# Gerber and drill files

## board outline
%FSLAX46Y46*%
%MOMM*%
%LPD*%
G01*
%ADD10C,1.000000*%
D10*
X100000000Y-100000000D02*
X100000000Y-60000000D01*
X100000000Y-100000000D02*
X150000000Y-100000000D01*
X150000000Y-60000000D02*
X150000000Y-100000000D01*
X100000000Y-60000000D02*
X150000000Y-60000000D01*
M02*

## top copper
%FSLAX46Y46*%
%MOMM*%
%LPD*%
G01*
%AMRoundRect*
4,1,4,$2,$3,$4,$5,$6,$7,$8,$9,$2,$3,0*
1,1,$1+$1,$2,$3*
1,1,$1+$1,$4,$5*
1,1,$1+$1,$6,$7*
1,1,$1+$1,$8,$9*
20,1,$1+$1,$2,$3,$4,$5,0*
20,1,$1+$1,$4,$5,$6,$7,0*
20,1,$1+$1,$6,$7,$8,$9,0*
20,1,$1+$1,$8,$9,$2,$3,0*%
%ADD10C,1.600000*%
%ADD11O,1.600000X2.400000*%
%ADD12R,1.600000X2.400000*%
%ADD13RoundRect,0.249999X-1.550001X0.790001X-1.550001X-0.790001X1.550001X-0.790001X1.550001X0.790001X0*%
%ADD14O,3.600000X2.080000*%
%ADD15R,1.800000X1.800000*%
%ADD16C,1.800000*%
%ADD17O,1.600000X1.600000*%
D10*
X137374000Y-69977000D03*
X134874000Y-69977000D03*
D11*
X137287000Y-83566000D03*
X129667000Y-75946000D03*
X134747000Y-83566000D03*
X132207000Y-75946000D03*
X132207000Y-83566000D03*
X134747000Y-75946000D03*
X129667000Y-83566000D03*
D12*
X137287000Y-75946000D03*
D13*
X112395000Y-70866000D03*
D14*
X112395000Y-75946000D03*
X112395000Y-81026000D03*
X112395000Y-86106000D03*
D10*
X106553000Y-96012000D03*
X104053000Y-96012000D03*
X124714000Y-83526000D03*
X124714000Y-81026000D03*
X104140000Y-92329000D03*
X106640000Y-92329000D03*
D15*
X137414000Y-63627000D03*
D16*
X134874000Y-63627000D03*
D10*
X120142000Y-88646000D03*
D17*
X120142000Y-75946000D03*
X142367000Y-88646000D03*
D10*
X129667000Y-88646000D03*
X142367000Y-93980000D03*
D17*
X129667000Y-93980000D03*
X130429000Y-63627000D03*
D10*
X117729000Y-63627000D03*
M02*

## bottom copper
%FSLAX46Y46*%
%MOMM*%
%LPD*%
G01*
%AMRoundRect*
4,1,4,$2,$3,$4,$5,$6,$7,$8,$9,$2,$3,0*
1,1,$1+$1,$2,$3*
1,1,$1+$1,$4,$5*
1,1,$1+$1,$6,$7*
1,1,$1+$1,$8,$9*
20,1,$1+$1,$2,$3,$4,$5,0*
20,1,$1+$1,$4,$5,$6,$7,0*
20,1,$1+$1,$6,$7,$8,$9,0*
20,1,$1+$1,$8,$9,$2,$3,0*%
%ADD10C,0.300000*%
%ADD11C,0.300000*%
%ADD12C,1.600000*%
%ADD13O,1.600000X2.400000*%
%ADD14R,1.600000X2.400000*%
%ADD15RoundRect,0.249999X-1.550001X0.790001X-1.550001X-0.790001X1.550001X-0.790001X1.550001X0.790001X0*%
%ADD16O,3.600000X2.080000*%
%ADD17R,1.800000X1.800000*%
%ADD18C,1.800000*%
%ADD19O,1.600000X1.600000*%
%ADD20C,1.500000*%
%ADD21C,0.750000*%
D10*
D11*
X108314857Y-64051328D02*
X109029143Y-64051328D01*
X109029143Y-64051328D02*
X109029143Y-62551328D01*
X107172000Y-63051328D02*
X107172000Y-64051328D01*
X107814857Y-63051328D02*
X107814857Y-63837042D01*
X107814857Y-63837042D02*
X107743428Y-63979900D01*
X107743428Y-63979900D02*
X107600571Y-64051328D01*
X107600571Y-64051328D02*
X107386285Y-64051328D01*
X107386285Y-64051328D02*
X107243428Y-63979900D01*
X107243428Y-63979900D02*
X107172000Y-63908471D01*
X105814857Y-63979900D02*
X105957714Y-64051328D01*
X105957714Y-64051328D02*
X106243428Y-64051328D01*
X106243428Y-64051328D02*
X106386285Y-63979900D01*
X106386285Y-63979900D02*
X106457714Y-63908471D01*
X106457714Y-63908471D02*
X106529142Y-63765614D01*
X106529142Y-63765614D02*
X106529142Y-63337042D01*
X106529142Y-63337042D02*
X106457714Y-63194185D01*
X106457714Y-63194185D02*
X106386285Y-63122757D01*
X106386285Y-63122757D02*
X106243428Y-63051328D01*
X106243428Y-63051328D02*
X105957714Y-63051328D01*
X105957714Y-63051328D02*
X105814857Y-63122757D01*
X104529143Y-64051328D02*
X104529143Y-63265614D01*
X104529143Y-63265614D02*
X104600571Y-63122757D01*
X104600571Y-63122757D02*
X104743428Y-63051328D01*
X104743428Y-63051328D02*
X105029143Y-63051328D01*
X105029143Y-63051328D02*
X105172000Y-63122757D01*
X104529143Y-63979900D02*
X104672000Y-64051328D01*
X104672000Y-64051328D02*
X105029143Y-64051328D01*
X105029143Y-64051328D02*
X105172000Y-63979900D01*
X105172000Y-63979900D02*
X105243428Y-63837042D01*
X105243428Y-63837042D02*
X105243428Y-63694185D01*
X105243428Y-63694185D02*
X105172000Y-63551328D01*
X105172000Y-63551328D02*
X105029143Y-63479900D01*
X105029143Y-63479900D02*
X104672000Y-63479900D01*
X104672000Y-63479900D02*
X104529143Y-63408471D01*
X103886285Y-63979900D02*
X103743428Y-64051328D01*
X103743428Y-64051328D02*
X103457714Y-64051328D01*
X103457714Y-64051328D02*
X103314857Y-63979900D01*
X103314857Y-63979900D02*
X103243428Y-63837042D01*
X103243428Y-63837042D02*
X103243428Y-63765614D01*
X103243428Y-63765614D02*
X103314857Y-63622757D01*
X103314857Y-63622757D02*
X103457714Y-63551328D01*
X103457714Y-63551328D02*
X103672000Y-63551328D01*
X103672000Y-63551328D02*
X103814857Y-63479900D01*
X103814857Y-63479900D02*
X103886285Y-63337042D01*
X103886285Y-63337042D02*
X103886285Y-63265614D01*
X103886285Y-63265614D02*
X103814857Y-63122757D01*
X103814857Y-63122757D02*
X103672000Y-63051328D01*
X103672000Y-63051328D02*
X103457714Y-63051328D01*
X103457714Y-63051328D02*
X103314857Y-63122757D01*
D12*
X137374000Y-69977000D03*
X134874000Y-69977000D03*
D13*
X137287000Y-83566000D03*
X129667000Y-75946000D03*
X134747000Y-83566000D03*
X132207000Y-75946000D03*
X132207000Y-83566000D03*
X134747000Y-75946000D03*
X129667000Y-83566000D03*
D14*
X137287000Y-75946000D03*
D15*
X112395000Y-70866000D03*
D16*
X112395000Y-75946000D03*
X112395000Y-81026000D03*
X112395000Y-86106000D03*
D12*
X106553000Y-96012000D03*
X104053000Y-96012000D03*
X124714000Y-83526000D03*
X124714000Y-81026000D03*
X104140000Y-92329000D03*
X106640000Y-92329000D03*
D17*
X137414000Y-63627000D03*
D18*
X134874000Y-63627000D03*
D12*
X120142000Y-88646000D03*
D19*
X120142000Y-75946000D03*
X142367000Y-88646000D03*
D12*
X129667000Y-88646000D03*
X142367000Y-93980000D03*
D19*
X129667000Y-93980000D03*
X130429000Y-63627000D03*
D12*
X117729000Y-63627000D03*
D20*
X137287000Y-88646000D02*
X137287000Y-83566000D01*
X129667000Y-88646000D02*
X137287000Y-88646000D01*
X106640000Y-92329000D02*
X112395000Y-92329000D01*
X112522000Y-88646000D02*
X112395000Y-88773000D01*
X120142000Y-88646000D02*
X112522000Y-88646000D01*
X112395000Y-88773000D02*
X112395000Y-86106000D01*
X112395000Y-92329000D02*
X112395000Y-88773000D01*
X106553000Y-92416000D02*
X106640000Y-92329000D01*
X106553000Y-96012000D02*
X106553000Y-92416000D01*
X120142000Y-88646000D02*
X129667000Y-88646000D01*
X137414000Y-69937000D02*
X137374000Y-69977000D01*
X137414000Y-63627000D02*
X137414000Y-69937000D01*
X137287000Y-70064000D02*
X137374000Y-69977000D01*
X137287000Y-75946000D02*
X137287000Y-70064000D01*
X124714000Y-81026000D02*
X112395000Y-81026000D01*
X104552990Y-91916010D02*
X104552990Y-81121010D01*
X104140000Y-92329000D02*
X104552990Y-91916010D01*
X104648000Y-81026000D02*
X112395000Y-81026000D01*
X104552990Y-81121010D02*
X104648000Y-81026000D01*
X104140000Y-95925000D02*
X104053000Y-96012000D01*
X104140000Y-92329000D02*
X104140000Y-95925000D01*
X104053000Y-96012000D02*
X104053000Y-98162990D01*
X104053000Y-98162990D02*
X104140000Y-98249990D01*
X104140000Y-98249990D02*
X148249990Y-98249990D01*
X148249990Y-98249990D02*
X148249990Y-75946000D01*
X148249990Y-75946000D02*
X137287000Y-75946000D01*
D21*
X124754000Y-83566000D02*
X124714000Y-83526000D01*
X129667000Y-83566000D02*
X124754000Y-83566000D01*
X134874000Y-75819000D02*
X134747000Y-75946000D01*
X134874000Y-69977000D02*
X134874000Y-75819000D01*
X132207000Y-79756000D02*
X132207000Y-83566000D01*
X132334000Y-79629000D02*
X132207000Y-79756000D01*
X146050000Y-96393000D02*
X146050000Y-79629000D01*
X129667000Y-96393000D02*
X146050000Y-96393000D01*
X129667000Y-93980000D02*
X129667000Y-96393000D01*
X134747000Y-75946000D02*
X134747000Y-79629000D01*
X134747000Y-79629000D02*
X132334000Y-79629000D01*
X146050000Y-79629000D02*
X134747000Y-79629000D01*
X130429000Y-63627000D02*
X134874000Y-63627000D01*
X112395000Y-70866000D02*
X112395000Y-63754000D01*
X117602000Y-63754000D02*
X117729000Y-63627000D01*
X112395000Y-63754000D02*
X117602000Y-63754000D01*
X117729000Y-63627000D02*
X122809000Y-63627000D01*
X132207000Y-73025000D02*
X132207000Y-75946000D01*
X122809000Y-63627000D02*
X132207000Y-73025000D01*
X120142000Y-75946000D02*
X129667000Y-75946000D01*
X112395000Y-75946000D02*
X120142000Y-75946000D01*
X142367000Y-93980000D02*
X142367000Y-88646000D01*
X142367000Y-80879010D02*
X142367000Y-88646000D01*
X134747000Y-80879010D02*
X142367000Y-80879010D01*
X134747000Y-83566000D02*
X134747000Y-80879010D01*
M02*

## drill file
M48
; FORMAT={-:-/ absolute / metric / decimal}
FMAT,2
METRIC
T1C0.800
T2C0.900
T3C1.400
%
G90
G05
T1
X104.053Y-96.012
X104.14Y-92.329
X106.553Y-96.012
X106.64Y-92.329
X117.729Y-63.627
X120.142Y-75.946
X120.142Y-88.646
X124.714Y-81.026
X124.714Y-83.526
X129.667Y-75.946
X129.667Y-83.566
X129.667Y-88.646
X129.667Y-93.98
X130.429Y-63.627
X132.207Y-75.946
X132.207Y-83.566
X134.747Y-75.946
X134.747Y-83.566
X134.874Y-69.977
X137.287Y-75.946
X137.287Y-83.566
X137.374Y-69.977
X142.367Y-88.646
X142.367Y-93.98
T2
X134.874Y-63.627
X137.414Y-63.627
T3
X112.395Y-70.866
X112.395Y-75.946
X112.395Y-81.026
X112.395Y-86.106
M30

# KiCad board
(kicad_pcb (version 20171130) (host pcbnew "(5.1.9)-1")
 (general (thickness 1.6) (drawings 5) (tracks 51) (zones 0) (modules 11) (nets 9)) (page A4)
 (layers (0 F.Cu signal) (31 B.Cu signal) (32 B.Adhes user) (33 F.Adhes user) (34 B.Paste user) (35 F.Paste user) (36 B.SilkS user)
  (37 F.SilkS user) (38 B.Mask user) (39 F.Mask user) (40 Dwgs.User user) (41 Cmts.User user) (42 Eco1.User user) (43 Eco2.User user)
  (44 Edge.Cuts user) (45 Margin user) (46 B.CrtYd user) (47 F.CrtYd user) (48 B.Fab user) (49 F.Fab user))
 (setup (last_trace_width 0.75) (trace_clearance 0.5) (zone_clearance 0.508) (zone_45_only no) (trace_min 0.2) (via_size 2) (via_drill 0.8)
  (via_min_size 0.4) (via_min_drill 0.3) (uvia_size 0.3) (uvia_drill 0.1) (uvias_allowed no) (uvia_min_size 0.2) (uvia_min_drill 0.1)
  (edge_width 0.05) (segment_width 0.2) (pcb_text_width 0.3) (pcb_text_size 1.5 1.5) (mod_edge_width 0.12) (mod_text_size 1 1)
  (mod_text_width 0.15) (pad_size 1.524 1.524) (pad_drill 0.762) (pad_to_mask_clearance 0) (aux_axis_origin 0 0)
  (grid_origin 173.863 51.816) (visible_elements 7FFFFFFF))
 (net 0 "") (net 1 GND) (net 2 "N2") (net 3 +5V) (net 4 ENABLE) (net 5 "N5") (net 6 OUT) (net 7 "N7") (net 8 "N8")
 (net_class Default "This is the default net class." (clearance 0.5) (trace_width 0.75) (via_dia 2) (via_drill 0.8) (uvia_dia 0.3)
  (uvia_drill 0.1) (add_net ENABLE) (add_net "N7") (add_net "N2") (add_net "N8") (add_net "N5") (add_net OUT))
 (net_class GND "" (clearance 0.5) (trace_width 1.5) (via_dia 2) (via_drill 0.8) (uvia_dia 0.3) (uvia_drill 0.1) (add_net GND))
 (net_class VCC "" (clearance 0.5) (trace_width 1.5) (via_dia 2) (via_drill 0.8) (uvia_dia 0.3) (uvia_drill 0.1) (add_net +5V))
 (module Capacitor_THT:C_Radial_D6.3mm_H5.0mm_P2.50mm (layer F.Cu) (at 134.874 69.977)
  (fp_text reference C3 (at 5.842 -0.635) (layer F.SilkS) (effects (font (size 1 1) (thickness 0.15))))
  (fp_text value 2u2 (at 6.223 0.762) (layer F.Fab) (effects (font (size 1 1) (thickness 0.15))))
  (pad 2 thru_hole circle (at 2.5 0) (size 1.6 1.6) (drill 0.8) (layers *.Cu *.Mask) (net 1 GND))
  (pad 1 thru_hole circle (at 0 0) (size 1.6 1.6) (drill 0.8) (layers *.Cu *.Mask) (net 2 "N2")))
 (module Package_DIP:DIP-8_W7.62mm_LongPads (layer F.Cu) (at 137.287 75.946 270)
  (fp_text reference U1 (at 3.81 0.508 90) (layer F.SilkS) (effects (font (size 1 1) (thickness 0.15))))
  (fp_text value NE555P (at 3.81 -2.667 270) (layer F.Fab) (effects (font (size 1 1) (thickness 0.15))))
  (pad 8 thru_hole oval (at 7.62 0 270) (size 2.4 1.6) (drill 0.8) (layers *.Cu *.Mask) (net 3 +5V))
  (pad 4 thru_hole oval (at 0 7.62 270) (size 2.4 1.6) (drill 0.8) (layers *.Cu *.Mask) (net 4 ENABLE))
  (pad 7 thru_hole oval (at 7.62 2.54 270) (size 2.4 1.6) (drill 0.8) (layers *.Cu *.Mask) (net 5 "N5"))
  (pad 3 thru_hole oval (at 0 5.08 270) (size 2.4 1.6) (drill 0.8) (layers *.Cu *.Mask) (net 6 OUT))
  (pad 6 thru_hole oval (at 7.62 5.08 270) (size 2.4 1.6) (drill 0.8) (layers *.Cu *.Mask) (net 2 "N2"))
  (pad 2 thru_hole oval (at 0 2.54 270) (size 2.4 1.6) (drill 0.8) (layers *.Cu *.Mask) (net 2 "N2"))
  (pad 5 thru_hole oval (at 7.62 7.62 270) (size 2.4 1.6) (drill 0.8) (layers *.Cu *.Mask) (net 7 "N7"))
  (pad 1 thru_hole rect (at 0 0 270) (size 2.4 1.6) (drill 0.8) (layers *.Cu *.Mask) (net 1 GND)))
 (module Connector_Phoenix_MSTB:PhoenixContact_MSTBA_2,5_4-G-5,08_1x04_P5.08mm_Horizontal (layer F.Cu) (at 112.395 70.866 270)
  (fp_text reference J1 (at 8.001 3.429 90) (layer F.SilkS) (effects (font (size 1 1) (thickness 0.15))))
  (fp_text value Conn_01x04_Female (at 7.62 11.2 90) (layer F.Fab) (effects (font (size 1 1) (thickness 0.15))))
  (pad 1 thru_hole roundrect (at 0 0 270) (size 2.08 3.6) (drill 1.4) (layers *.Cu *.Mask) (roundrect_rratio 0.120192) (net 6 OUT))
  (pad 2 thru_hole oval (at 5.08 0 270) (size 2.08 3.6) (drill 1.4) (layers *.Cu *.Mask) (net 4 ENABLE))
  (pad 3 thru_hole oval (at 10.16 0 270) (size 2.08 3.6) (drill 1.4) (layers *.Cu *.Mask) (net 1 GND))
  (pad 4 thru_hole oval (at 15.24 0 270) (size 2.08 3.6) (drill 1.4) (layers *.Cu *.Mask) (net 3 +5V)))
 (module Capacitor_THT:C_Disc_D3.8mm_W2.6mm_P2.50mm (layer F.Cu) (at 106.553 96.012 180)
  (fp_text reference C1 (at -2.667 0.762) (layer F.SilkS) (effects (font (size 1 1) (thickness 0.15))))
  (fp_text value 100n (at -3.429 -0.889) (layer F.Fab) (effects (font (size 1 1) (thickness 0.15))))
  (pad 1 thru_hole circle (at 0 0 180) (size 1.6 1.6) (drill 0.8) (layers *.Cu *.Mask) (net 3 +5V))
  (pad 2 thru_hole circle (at 2.5 0 180) (size 1.6 1.6) (drill 0.8) (layers *.Cu *.Mask) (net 1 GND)))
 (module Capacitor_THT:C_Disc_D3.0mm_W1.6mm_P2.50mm (layer F.Cu) (at 124.714 83.526 90)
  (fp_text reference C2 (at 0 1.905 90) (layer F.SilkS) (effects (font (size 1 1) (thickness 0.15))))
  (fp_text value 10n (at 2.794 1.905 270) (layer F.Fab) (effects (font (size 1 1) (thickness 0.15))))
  (pad 1 thru_hole circle (at 0 0 90) (size 1.6 1.6) (drill 0.8) (layers *.Cu *.Mask) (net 7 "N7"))
  (pad 2 thru_hole circle (at 2.5 0 90) (size 1.6 1.6) (drill 0.8) (layers *.Cu *.Mask) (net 1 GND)))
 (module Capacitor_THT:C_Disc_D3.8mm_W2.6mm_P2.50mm (layer F.Cu) (at 106.64 92.329 180)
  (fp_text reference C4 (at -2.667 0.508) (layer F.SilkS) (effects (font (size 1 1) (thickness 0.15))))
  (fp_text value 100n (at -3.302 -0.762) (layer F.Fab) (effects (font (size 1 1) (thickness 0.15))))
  (pad 2 thru_hole circle (at 2.5 0 180) (size 1.6 1.6) (drill 0.8) (layers *.Cu *.Mask) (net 1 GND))
  (pad 1 thru_hole circle (at 0 0 180) (size 1.6 1.6) (drill 0.8) (layers *.Cu *.Mask) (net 3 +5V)))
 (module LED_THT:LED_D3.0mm (layer F.Cu) (at 137.414 63.627 180)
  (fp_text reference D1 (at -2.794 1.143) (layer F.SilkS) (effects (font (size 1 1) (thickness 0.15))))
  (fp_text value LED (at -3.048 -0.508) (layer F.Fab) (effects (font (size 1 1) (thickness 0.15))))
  (pad 1 thru_hole rect (at 0 0 180) (size 1.8 1.8) (drill 0.9) (layers *.Cu *.Mask) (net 1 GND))
  (pad 2 thru_hole circle (at 2.54 0 180) (size 1.8 1.8) (drill 0.9) (layers *.Cu *.Mask) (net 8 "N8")))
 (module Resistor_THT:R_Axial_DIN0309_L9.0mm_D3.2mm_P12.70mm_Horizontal (layer F.Cu) (at 120.142 88.646 90)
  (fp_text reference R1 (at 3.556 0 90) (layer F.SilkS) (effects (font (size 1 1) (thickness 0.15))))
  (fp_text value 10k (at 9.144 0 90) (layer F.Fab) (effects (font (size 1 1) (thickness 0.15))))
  (pad 1 thru_hole circle (at 0 0 90) (size 1.6 1.6) (drill 0.8) (layers *.Cu *.Mask) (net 3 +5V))
  (pad 2 thru_hole oval (at 12.7 0 90) (size 1.6 1.6) (drill 0.8) (layers *.Cu *.Mask) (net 4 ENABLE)))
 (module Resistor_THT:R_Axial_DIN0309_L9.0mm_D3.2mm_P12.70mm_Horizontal (layer F.Cu) (at 129.667 88.646)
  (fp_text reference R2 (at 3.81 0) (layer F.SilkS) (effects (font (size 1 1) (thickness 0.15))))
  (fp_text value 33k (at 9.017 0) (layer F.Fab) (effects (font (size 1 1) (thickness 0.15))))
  (pad 2 thru_hole oval (at 12.7 0) (size 1.6 1.6) (drill 0.8) (layers *.Cu *.Mask) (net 5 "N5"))
  (pad 1 thru_hole circle (at 0 0) (size 1.6 1.6) (drill 0.8) (layers *.Cu *.Mask) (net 3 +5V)))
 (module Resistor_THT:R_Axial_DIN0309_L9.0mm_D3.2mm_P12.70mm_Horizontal (layer F.Cu) (at 142.367 93.98 180)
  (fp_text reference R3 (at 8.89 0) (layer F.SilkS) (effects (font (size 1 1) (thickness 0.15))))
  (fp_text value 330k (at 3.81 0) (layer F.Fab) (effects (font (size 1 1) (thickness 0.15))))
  (pad 1 thru_hole circle (at 0 0 180) (size 1.6 1.6) (drill 0.8) (layers *.Cu *.Mask) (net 5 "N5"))
  (pad 2 thru_hole oval (at 12.7 0 180) (size 1.6 1.6) (drill 0.8) (layers *.Cu *.Mask) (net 2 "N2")))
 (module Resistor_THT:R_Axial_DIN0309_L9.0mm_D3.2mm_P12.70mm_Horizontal (layer F.Cu) (at 117.729 63.627)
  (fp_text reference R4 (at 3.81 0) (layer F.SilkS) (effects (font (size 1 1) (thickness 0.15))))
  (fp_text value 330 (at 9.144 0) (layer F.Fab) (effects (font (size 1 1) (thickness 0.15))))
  (pad 2 thru_hole oval (at 12.7 0) (size 1.6 1.6) (drill 0.8) (layers *.Cu *.Mask) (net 8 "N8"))
  (pad 1 thru_hole circle (at 0 0) (size 1.6 1.6) (drill 0.8) (layers *.Cu *.Mask) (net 6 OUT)))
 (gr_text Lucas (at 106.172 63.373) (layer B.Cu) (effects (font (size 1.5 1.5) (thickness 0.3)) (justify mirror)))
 (gr_line (start 100 100) (end 100 60) (layer Edge.Cuts) (width 1))
 (gr_line (start 100 100) (end 150 100) (layer Edge.Cuts) (width 1))
 (gr_line (start 150 60) (end 150 100) (layer Edge.Cuts) (width 1))
 (gr_line (start 100 60) (end 150 60) (layer Edge.Cuts) (width 1))
 (segment (start 137.287 88.646) (end 137.287 83.566) (width 1.5) (layer B.Cu) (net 3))
 (segment (start 129.667 88.646) (end 137.287 88.646) (width 1.5) (layer B.Cu) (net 3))
 (segment (start 106.64 92.329) (end 112.395 92.329) (width 1.5) (layer B.Cu) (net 3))
 (segment (start 112.522 88.646) (end 112.395 88.773) (width 1.5) (layer B.Cu) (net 3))
 (segment (start 120.142 88.646) (end 112.522 88.646) (width 1.5) (layer B.Cu) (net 3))
 (segment (start 112.395 88.773) (end 112.395 86.106) (width 1.5) (layer B.Cu) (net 3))
 (segment (start 112.395 92.329) (end 112.395 88.773) (width 1.5) (layer B.Cu) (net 3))
 (segment (start 106.553 92.416) (end 106.64 92.329) (width 1.5) (layer B.Cu) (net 3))
 (segment (start 106.553 96.012) (end 106.553 92.416) (width 1.5) (layer B.Cu) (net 3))
 (segment (start 120.142 88.646) (end 129.667 88.646) (width 1.5) (layer B.Cu) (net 3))
 (segment (start 137.414 69.937) (end 137.374 69.977) (width 1.5) (layer B.Cu) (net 1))
 (segment (start 137.414 63.627) (end 137.414 69.937) (width 1.5) (layer B.Cu) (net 1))
 (segment (start 137.287 70.064) (end 137.374 69.977) (width 1.5) (layer B.Cu) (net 1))
 (segment (start 137.287 75.946) (end 137.287 70.064) (width 1.5) (layer B.Cu) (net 1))
 (segment (start 124.714 81.026) (end 112.395 81.026) (width 1.5) (layer B.Cu) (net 1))
 (segment (start 104.55299 91.91601) (end 104.55299 81.12101) (width 1.5) (layer B.Cu) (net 1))
 (segment (start 104.14 92.329) (end 104.55299 91.91601) (width 1.5) (layer B.Cu) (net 1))
 (segment (start 104.648 81.026) (end 112.395 81.026) (width 1.5) (layer B.Cu) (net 1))
 (segment (start 104.55299 81.12101) (end 104.648 81.026) (width 1.5) (layer B.Cu) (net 1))
 (segment (start 104.14 95.925) (end 104.053 96.012) (width 1.5) (layer B.Cu) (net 1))
 (segment (start 104.14 92.329) (end 104.14 95.925) (width 1.5) (layer B.Cu) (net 1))
 (segment (start 104.053 96.012) (end 104.053 98.16299) (width 1.5) (layer B.Cu) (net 1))
 (segment (start 104.053 98.16299) (end 104.14 98.24999) (width 1.5) (layer B.Cu) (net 1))
 (segment (start 104.14 98.24999) (end 148.24999 98.24999) (width 1.5) (layer B.Cu) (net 1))
 (segment (start 148.24999 98.24999) (end 148.24999 75.946) (width 1.5) (layer B.Cu) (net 1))
 (segment (start 148.24999 75.946) (end 137.287 75.946) (width 1.5) (layer B.Cu) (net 1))
 (segment (start 124.754 83.566) (end 124.714 83.526) (width 0.75) (layer B.Cu) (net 7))
 (segment (start 129.667 83.566) (end 124.754 83.566) (width 0.75) (layer B.Cu) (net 7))
 (segment (start 134.874 75.819) (end 134.747 75.946) (width 0.75) (layer B.Cu) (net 2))
 (segment (start 134.874 69.977) (end 134.874 75.819) (width 0.75) (layer B.Cu) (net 2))
 (segment (start 132.207 79.756) (end 132.207 83.566) (width 0.75) (layer B.Cu) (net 2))
 (segment (start 132.334 79.629) (end 132.207 79.756) (width 0.75) (layer B.Cu) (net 2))
 (segment (start 146.05 96.393) (end 146.05 79.629) (width 0.75) (layer B.Cu) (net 2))
 (segment (start 129.667 96.393) (end 146.05 96.393) (width 0.75) (layer B.Cu) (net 2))
 (segment (start 129.667 93.98) (end 129.667 96.393) (width 0.75) (layer B.Cu) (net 2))
 (segment (start 134.747 75.946) (end 134.747 79.629) (width 0.75) (layer B.Cu) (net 2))
 (segment (start 134.747 79.629) (end 132.334 79.629) (width 0.75) (layer B.Cu) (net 2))
 (segment (start 146.05 79.629) (end 134.747 79.629) (width 0.75) (layer B.Cu) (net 2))
 (segment (start 130.429 63.627) (end 134.874 63.627) (width 0.75) (layer B.Cu) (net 8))
 (segment (start 112.395 70.866) (end 112.395 63.754) (width 0.75) (layer B.Cu) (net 6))
 (segment (start 117.602 63.754) (end 117.729 63.627) (width 0.75) (layer B.Cu) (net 6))
 (segment (start 112.395 63.754) (end 117.602 63.754) (width 0.75) (layer B.Cu) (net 6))
 (segment (start 117.729 63.627) (end 122.809 63.627) (width 0.75) (layer B.Cu) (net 6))
 (segment (start 132.207 73.025) (end 132.207 75.946) (width 0.75) (layer B.Cu) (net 6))
 (segment (start 122.809 63.627) (end 132.207 73.025) (width 0.75) (layer B.Cu) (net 6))
 (segment (start 120.142 75.946) (end 129.667 75.946) (width 0.75) (layer B.Cu) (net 4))
 (segment (start 112.395 75.946) (end 120.142 75.946) (width 0.75) (layer B.Cu) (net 4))
 (segment (start 142.367 93.98) (end 142.367 88.646) (width 0.75) (layer B.Cu) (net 5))
 (segment (start 142.367 80.87901) (end 142.367 88.646) (width 0.75) (layer B.Cu) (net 5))
 (segment (start 134.747 80.87901) (end 142.367 80.87901) (width 0.75) (layer B.Cu) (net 5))
 (segment (start 134.747 83.566) (end 134.747 80.87901) (width 0.75) (layer B.Cu) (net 5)))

